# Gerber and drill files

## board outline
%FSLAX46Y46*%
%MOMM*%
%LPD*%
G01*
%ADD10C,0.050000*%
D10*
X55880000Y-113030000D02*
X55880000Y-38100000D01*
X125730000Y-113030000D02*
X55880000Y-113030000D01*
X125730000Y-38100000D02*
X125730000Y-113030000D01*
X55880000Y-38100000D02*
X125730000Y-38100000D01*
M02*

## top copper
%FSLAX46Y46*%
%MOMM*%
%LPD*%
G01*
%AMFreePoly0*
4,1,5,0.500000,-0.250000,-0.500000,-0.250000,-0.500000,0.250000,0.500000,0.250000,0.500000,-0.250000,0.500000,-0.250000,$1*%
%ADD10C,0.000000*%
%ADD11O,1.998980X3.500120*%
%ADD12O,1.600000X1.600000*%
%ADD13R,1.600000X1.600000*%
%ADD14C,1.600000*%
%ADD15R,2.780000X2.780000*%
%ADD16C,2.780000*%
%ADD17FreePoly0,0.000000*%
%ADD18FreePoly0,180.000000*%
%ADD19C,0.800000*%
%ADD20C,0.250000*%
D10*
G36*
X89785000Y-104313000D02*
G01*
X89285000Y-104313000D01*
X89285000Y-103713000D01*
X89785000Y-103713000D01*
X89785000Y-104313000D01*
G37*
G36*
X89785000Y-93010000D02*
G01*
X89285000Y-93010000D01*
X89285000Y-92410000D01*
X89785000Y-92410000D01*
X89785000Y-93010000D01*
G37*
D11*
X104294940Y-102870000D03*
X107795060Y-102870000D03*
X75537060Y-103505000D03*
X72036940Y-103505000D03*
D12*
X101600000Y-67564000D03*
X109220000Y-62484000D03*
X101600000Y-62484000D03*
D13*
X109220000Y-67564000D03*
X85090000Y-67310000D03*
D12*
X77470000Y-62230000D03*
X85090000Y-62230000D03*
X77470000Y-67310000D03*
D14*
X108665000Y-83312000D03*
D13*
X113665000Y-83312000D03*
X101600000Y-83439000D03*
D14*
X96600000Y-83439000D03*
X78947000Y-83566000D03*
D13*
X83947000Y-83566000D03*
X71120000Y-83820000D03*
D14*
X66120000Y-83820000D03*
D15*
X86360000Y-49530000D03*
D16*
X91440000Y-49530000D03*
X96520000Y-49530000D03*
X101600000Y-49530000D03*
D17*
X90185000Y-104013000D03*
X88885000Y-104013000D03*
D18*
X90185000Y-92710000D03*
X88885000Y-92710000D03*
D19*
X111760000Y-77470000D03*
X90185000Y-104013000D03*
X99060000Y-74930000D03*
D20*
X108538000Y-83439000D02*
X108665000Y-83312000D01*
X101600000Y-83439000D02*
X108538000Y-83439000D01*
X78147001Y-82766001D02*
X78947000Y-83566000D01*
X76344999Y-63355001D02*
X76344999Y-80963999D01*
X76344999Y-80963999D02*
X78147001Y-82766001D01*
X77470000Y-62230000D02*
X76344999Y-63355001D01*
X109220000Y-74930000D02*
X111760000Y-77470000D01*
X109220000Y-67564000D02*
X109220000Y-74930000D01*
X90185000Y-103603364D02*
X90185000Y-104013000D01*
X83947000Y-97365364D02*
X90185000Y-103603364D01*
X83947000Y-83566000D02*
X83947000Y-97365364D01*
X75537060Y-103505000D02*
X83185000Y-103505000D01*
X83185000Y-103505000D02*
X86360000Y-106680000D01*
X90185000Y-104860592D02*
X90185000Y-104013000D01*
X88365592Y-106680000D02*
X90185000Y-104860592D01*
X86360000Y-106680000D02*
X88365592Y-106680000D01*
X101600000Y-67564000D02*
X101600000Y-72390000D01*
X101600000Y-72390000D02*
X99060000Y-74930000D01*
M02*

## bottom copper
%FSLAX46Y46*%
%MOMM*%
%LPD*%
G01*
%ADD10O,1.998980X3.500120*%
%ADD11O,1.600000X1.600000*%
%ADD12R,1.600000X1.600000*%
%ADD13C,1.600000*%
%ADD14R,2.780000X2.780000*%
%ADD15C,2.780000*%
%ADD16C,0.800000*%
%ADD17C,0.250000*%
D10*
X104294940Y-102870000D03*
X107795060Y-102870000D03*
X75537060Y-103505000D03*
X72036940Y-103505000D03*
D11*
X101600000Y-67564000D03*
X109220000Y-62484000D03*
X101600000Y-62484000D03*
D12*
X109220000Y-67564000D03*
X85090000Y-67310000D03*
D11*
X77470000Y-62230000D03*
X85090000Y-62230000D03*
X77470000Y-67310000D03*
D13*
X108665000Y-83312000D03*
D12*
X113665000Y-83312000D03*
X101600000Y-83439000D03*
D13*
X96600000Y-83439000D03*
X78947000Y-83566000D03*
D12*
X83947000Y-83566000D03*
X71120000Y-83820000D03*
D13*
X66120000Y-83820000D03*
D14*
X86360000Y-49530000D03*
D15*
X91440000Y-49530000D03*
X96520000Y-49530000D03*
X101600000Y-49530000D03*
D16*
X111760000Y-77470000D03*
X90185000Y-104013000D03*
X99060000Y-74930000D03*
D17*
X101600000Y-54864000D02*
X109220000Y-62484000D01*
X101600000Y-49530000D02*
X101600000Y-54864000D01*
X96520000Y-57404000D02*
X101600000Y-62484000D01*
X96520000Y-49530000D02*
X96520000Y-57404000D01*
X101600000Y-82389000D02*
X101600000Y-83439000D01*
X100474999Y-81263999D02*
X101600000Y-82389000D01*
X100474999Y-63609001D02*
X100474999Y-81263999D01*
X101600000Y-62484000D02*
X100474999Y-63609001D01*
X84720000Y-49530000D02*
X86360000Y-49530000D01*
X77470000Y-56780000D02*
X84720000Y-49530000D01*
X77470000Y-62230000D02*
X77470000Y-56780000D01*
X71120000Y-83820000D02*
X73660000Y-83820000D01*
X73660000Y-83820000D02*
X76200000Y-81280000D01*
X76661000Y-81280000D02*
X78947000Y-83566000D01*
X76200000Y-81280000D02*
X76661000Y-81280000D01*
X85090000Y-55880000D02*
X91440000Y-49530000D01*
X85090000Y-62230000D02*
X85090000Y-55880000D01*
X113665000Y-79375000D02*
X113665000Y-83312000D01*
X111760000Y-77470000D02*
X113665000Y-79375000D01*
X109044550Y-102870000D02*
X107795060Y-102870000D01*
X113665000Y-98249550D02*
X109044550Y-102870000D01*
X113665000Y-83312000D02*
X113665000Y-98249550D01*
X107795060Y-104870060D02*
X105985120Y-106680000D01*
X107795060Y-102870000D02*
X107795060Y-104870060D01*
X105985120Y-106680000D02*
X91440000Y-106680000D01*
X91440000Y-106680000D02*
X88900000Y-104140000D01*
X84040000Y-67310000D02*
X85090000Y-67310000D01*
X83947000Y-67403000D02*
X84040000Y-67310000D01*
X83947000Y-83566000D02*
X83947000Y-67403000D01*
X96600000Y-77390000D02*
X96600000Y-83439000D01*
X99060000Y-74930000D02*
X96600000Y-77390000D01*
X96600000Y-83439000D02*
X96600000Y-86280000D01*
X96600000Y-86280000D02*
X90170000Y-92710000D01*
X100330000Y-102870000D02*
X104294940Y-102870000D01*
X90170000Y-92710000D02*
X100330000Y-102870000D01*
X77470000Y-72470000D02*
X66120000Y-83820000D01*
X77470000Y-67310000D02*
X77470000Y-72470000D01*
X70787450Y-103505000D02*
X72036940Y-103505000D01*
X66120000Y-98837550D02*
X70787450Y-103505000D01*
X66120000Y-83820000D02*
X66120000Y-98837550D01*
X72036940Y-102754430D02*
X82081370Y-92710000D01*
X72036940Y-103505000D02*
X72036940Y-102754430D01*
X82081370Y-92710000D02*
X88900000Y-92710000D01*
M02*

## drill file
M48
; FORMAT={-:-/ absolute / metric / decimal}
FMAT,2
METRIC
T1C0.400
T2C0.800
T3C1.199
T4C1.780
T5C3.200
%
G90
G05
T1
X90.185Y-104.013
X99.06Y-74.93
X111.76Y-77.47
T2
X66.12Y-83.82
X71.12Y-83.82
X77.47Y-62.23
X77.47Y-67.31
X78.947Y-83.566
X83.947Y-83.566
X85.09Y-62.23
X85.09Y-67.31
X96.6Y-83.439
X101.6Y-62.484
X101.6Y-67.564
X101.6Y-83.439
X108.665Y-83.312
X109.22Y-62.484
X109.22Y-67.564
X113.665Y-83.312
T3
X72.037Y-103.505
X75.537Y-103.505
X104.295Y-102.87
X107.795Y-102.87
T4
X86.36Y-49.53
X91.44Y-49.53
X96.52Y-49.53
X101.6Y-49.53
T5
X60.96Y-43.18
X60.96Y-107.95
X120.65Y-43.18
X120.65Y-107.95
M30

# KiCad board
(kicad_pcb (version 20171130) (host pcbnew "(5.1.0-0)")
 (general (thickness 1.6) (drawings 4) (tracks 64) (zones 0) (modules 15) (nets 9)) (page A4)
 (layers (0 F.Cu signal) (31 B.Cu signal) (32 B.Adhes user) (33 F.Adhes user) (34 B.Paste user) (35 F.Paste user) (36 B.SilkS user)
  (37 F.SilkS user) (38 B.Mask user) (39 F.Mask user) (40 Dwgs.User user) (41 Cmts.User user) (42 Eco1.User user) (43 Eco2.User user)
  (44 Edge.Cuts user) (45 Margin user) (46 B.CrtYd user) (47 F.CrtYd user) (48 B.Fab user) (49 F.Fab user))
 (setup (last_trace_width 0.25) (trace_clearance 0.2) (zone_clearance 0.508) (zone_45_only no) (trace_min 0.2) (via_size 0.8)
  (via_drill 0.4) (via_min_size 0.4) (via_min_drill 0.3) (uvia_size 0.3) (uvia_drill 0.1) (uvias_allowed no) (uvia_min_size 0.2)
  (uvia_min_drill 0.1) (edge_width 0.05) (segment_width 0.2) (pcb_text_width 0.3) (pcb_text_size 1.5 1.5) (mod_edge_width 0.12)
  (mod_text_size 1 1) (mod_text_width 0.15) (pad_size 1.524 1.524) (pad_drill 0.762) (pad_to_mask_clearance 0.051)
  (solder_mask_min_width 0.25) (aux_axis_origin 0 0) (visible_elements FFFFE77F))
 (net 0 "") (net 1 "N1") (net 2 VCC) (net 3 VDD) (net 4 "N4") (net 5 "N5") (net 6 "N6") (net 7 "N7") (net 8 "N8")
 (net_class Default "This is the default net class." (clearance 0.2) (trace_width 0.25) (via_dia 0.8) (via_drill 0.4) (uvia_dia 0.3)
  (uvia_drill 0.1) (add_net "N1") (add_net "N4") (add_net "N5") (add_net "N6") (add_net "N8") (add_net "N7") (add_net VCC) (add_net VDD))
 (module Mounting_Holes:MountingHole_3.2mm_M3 (layer F.Cu) (at 120.65 43.18)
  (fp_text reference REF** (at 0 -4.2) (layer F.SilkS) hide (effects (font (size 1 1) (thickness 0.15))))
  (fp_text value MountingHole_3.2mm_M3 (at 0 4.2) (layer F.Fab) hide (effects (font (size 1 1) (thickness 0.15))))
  (pad 1 np_thru_hole circle (at 0 0) (size 3.2 3.2) (drill 3.2) (layers *.Cu *.Mask)))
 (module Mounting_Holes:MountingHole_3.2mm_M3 (layer F.Cu) (at 120.65 107.95)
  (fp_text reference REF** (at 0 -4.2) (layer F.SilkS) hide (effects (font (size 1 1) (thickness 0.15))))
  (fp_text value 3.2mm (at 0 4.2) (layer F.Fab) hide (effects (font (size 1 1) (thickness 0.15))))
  (pad 1 np_thru_hole circle (at 0 0) (size 3.2 3.2) (drill 3.2) (layers *.Cu *.Mask)))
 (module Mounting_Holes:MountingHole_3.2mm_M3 (layer F.Cu) (at 60.96 107.95)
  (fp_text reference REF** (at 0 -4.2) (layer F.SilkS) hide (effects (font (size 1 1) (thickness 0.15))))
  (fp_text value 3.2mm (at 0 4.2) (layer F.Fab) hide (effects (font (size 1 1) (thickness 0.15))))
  (pad 1 np_thru_hole circle (at 0 0) (size 3.2 3.2) (drill 3.2) (layers *.Cu *.Mask)))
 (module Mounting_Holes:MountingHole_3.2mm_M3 (layer F.Cu) (at 60.96 43.18)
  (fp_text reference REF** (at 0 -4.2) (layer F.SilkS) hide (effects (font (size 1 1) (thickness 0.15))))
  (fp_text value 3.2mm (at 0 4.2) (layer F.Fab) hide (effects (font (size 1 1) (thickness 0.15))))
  (pad 1 np_thru_hole circle (at 0 0) (size 3.2 3.2) (drill 3.2) (layers *.Cu *.Mask)))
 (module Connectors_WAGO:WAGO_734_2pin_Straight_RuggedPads (layer F.Cu) (at 106.045 102.87)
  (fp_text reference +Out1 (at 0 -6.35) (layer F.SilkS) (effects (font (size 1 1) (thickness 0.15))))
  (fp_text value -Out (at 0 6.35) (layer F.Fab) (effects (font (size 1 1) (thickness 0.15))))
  (pad 1 thru_hole oval (at -1.75006 0) (size 1.99898 3.50012) (drill 1.19888) (layers *.Cu *.Mask) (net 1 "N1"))
  (pad 2 thru_hole oval (at 1.75006 0) (size 1.99898 3.50012) (drill 1.19888) (layers *.Cu *.Mask) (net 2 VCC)))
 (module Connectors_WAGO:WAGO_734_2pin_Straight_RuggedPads (layer F.Cu) (at 73.787 103.505)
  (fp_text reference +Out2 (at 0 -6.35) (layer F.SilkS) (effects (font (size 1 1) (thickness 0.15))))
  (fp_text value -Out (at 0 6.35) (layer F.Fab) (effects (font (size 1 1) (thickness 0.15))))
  (pad 2 thru_hole oval (at 1.75006 0) (size 1.99898 3.50012) (drill 1.19888) (layers *.Cu *.Mask) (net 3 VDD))
  (pad 1 thru_hole oval (at -1.75006 0) (size 1.99898 3.50012) (drill 1.19888) (layers *.Cu *.Mask) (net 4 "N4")))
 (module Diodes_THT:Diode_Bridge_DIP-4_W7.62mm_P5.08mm (layer F.Cu) (at 109.22 67.564 180)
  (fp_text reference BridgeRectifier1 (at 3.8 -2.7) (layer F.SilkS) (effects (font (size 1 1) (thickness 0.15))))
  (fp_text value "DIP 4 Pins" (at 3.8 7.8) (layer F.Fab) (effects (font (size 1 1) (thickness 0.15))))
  (pad 4 thru_hole oval (at 7.62 0 180) (size 1.6 1.6) (drill 0.8) (layers *.Cu *.Mask) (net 1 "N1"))
  (pad 2 thru_hole oval (at 0 5.08 180) (size 1.6 1.6) (drill 0.8) (layers *.Cu *.Mask) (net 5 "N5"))
  (pad 3 thru_hole oval (at 7.62 5.08 180) (size 1.6 1.6) (drill 0.8) (layers *.Cu *.Mask) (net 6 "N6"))
  (pad 1 thru_hole rect (at 0 0 180) (size 1.6 1.6) (drill 0.8) (layers *.Cu *.Mask) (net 2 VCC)))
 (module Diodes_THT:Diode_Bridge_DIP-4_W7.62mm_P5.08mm (layer F.Cu) (at 85.09 67.31 180)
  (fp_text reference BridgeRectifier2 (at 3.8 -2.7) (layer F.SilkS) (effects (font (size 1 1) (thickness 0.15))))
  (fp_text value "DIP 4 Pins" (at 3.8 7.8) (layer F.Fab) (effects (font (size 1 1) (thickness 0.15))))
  (pad 1 thru_hole rect (at 0 0 180) (size 1.6 1.6) (drill 0.8) (layers *.Cu *.Mask) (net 3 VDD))
  (pad 3 thru_hole oval (at 7.62 5.08 180) (size 1.6 1.6) (drill 0.8) (layers *.Cu *.Mask) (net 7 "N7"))
  (pad 2 thru_hole oval (at 0 5.08 180) (size 1.6 1.6) (drill 0.8) (layers *.Cu *.Mask) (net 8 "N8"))
  (pad 4 thru_hole oval (at 7.62 0 180) (size 1.6 1.6) (drill 0.8) (layers *.Cu *.Mask) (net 4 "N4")))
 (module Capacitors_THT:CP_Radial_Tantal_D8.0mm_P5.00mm (layer F.Cu) (at 113.665 83.312 180)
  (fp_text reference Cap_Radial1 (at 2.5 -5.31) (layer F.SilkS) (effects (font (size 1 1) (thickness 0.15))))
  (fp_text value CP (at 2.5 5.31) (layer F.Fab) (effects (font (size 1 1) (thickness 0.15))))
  (pad 2 thru_hole circle (at 5 0 180) (size 1.6 1.6) (drill 0.8) (layers *.Cu *.Mask) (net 6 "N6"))
  (pad 1 thru_hole rect (at 0 0 180) (size 1.6 1.6) (drill 0.8) (layers *.Cu *.Mask) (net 2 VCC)))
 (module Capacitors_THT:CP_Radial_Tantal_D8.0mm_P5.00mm (layer F.Cu) (at 101.6 83.439 180)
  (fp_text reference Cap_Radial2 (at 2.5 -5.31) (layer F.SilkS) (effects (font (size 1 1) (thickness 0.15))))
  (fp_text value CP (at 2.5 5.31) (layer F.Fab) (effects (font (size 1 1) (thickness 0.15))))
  (pad 1 thru_hole rect (at 0 0 180) (size 1.6 1.6) (drill 0.8) (layers *.Cu *.Mask) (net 6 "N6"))
  (pad 2 thru_hole circle (at 5 0 180) (size 1.6 1.6) (drill 0.8) (layers *.Cu *.Mask) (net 1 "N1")))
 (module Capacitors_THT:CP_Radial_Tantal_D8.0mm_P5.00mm (layer F.Cu) (at 83.947 83.566 180)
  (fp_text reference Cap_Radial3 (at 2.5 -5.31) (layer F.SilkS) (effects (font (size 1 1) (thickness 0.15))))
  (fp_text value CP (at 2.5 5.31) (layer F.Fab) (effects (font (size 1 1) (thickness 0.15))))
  (pad 2 thru_hole circle (at 5 0 180) (size 1.6 1.6) (drill 0.8) (layers *.Cu *.Mask) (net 7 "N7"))
  (pad 1 thru_hole rect (at 0 0 180) (size 1.6 1.6) (drill 0.8) (layers *.Cu *.Mask) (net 3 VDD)))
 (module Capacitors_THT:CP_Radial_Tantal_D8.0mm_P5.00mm (layer F.Cu) (at 71.12 83.82 180)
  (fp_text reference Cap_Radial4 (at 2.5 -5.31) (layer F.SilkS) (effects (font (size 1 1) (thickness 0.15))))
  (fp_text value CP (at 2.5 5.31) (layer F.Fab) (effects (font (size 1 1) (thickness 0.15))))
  (pad 1 thru_hole rect (at 0 0 180) (size 1.6 1.6) (drill 0.8) (layers *.Cu *.Mask) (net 7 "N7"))
  (pad 2 thru_hole circle (at 5 0 180) (size 1.6 1.6) (drill 0.8) (layers *.Cu *.Mask) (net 4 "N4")))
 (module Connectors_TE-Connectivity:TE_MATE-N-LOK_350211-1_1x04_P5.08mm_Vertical (layer F.Cu) (at 86.36 49.53)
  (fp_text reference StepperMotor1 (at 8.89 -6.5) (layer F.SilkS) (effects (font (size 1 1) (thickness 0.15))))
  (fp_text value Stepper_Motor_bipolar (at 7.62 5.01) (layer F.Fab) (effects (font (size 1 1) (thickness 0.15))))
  (pad 1 thru_hole rect (at 0 0) (size 2.78 2.78) (drill 1.78) (layers *.Cu *.Mask) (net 7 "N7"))
  (pad 2 thru_hole circle (at 5.08 0) (size 2.78 2.78) (drill 1.78) (layers *.Cu *.Mask) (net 8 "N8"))
  (pad 3 thru_hole circle (at 10.16 0) (size 2.78 2.78) (drill 1.78) (layers *.Cu *.Mask) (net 6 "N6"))
  (pad 4 thru_hole circle (at 15.24 0) (size 2.78 2.78) (drill 1.78) (layers *.Cu *.Mask) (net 5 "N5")))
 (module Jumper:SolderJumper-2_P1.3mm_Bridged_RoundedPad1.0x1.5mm (layer F.Cu) (at 89.535 104.013)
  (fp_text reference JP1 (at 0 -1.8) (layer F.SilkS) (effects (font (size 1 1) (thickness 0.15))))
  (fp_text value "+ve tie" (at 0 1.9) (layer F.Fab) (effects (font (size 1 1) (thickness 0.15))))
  (fp_poly (pts (xy 0.25 -0.3) (xy -0.25 -0.3) (xy -0.25 0.3) (xy 0.25 0.3)) (layer F.Cu) (width 0))
  (pad 2 smd custom (at 0.65 0) (size 1 0.5) (layers F.Cu F.Mask) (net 3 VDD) (zone_connect 2) (options (clearance outline) (anchor rect))
   (primitives))
  (pad 1 smd custom (at -0.65 0) (size 1 0.5) (layers F.Cu F.Mask) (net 2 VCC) (zone_connect 2) (options (clearance outline) (anchor rect))
   (primitives)))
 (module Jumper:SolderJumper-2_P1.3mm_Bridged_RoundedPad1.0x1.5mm (layer F.Cu) (at 89.535 92.71 180)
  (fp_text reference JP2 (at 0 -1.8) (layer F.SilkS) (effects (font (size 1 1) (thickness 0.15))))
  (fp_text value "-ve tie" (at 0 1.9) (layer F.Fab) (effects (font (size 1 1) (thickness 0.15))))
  (fp_poly (pts (xy 0.25 -0.3) (xy -0.25 -0.3) (xy -0.25 0.3) (xy 0.25 0.3)) (layer F.Cu) (width 0))
  (pad 1 smd custom (at -0.65 0 180) (size 1 0.5) (layers F.Cu F.Mask) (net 1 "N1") (zone_connect 2)
   (options (clearance outline) (anchor rect)) (primitives))
  (pad 2 smd custom (at 0.65 0 180) (size 1 0.5) (layers F.Cu F.Mask) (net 4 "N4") (zone_connect 2)
   (options (clearance outline) (anchor rect)) (primitives)))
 (gr_line (start 55.88 113.03) (end 55.88 38.1) (layer Edge.Cuts) (width 0.05))
 (gr_line (start 125.73 113.03) (end 55.88 113.03) (layer Edge.Cuts) (width 0.05))
 (gr_line (start 125.73 38.1) (end 125.73 113.03) (layer Edge.Cuts) (width 0.05))
 (gr_line (start 55.88 38.1) (end 125.73 38.1) (layer Edge.Cuts) (width 0.05))
 (segment (start 101.6 54.864) (end 109.22 62.484) (width 0.25) (layer B.Cu) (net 5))
 (segment (start 101.6 49.53) (end 101.6 54.864) (width 0.25) (layer B.Cu) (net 5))
 (segment (start 96.52 57.404) (end 101.6 62.484) (width 0.25) (layer B.Cu) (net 6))
 (segment (start 96.52 49.53) (end 96.52 57.404) (width 0.25) (layer B.Cu) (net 6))
 (segment (start 101.6 82.389) (end 101.6 83.439) (width 0.25) (layer B.Cu) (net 6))
 (segment (start 100.474999 81.263999) (end 101.6 82.389) (width 0.25) (layer B.Cu) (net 6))
 (segment (start 100.474999 63.609001) (end 100.474999 81.263999) (width 0.25) (layer B.Cu) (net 6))
 (segment (start 101.6 62.484) (end 100.474999 63.609001) (width 0.25) (layer B.Cu) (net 6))
 (segment (start 108.538 83.439) (end 108.665 83.312) (width 0.25) (layer F.Cu) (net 6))
 (segment (start 101.6 83.439) (end 108.538 83.439) (width 0.25) (layer F.Cu) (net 6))
 (segment (start 84.72 49.53) (end 86.36 49.53) (width 0.25) (layer B.Cu) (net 7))
 (segment (start 77.47 56.78) (end 84.72 49.53) (width 0.25) (layer B.Cu) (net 7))
 (segment (start 77.47 62.23) (end 77.47 56.78) (width 0.25) (layer B.Cu) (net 7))
 (segment (start 78.147001 82.766001) (end 78.947 83.566) (width 0.25) (layer F.Cu) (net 7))
 (segment (start 76.344999 63.355001) (end 76.344999 80.963999) (width 0.25) (layer F.Cu) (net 7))
 (segment (start 76.344999 80.963999) (end 78.147001 82.766001) (width 0.25) (layer F.Cu) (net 7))
 (segment (start 77.47 62.23) (end 76.344999 63.355001) (width 0.25) (layer F.Cu) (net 7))
 (segment (start 71.12 83.82) (end 73.66 83.82) (width 0.25) (layer B.Cu) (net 7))
 (segment (start 73.66 83.82) (end 76.2 81.28) (width 0.25) (layer B.Cu) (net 7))
 (segment (start 76.661 81.28) (end 78.947 83.566) (width 0.25) (layer B.Cu) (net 7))
 (segment (start 76.2 81.28) (end 76.661 81.28) (width 0.25) (layer B.Cu) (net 7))
 (segment (start 85.09 55.88) (end 91.44 49.53) (width 0.25) (layer B.Cu) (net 8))
 (segment (start 85.09 62.23) (end 85.09 55.88) (width 0.25) (layer B.Cu) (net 8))
 (via (at 111.76 77.47) (size 0.8) (drill 0.4) (layers F.Cu B.Cu) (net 2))
 (segment (start 109.22 74.93) (end 111.76 77.47) (width 0.25) (layer F.Cu) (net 2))
 (segment (start 109.22 67.564) (end 109.22 74.93) (width 0.25) (layer F.Cu) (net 2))
 (segment (start 113.665 79.375) (end 113.665 83.312) (width 0.25) (layer B.Cu) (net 2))
 (segment (start 111.76 77.47) (end 113.665 79.375) (width 0.25) (layer B.Cu) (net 2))
 (segment (start 109.04455 102.87) (end 107.79506 102.87) (width 0.25) (layer B.Cu) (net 2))
 (segment (start 113.665 98.24955) (end 109.04455 102.87) (width 0.25) (layer B.Cu) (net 2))
 (segment (start 113.665 83.312) (end 113.665 98.24955) (width 0.25) (layer B.Cu) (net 2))
 (segment (start 107.79506 104.87006) (end 105.98512 106.68) (width 0.25) (layer B.Cu) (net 2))
 (segment (start 107.79506 102.87) (end 107.79506 104.87006) (width 0.25) (layer B.Cu) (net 2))
 (segment (start 105.98512 106.68) (end 91.44 106.68) (width 0.25) (layer B.Cu) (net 2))
 (segment (start 91.44 106.68) (end 88.9 104.14) (width 0.25) (layer B.Cu) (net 2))
 (segment (start 84.04 67.31) (end 85.09 67.31) (width 0.25) (layer B.Cu) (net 3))
 (segment (start 83.947 67.403) (end 84.04 67.31) (width 0.25) (layer B.Cu) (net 3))
 (segment (start 83.947 83.566) (end 83.947 67.403) (width 0.25) (layer B.Cu) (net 3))
 (segment (start 90.185 103.603364) (end 90.185 104.013) (width 0.25) (layer F.Cu) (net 3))
 (segment (start 83.947 97.365364) (end 90.185 103.603364) (width 0.25) (layer F.Cu) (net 3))
 (segment (start 83.947 83.566) (end 83.947 97.365364) (width 0.25) (layer F.Cu) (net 3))
 (segment (start 75.53706 103.505) (end 83.185 103.505) (width 0.25) (layer F.Cu) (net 3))
 (segment (start 83.185 103.505) (end 86.36 106.68) (width 0.25) (layer F.Cu) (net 3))
 (segment (start 90.185 104.860592) (end 90.185 104.013) (width 0.25) (layer F.Cu) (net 3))
 (via (at 90.185 104.013) (size 0.8) (drill 0.4) (layers F.Cu B.Cu) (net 3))
 (segment (start 88.365592 106.68) (end 90.185 104.860592) (width 0.25) (layer F.Cu) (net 3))
 (segment (start 86.36 106.68) (end 88.365592 106.68) (width 0.25) (layer F.Cu) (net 3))
 (segment (start 101.6 67.564) (end 101.6 72.39) (width 0.25) (layer F.Cu) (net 1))
 (via (at 99.06 74.93) (size 0.8) (drill 0.4) (layers F.Cu B.Cu) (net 1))
 (segment (start 101.6 72.39) (end 99.06 74.93) (width 0.25) (layer F.Cu) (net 1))
 (segment (start 96.6 77.39) (end 96.6 83.439) (width 0.25) (layer B.Cu) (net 1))
 (segment (start 99.06 74.93) (end 96.6 77.39) (width 0.25) (layer B.Cu) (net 1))
 (segment (start 96.6 83.439) (end 96.6 86.28) (width 0.25) (layer B.Cu) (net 1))
 (segment (start 96.6 86.28) (end 90.17 92.71) (width 0.25) (layer B.Cu) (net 1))
 (segment (start 100.33 102.87) (end 104.29494 102.87) (width 0.25) (layer B.Cu) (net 1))
 (segment (start 90.17 92.71) (end 100.33 102.87) (width 0.25) (layer B.Cu) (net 1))
 (segment (start 77.47 72.47) (end 66.12 83.82) (width 0.25) (layer B.Cu) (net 4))
 (segment (start 77.47 67.31) (end 77.47 72.47) (width 0.25) (layer B.Cu) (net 4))
 (segment (start 70.78745 103.505) (end 72.03694 103.505) (width 0.25) (layer B.Cu) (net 4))
 (segment (start 66.12 98.83755) (end 70.78745 103.505) (width 0.25) (layer B.Cu) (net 4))
 (segment (start 66.12 83.82) (end 66.12 98.83755) (width 0.25) (layer B.Cu) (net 4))
 (segment (start 72.03694 102.75443) (end 82.08137 92.71) (width 0.25) (layer B.Cu) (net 4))
 (segment (start 72.03694 103.505) (end 72.03694 102.75443) (width 0.25) (layer B.Cu) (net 4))
 (segment (start 82.08137 92.71) (end 88.9 92.71) (width 0.25) (layer B.Cu) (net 4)))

